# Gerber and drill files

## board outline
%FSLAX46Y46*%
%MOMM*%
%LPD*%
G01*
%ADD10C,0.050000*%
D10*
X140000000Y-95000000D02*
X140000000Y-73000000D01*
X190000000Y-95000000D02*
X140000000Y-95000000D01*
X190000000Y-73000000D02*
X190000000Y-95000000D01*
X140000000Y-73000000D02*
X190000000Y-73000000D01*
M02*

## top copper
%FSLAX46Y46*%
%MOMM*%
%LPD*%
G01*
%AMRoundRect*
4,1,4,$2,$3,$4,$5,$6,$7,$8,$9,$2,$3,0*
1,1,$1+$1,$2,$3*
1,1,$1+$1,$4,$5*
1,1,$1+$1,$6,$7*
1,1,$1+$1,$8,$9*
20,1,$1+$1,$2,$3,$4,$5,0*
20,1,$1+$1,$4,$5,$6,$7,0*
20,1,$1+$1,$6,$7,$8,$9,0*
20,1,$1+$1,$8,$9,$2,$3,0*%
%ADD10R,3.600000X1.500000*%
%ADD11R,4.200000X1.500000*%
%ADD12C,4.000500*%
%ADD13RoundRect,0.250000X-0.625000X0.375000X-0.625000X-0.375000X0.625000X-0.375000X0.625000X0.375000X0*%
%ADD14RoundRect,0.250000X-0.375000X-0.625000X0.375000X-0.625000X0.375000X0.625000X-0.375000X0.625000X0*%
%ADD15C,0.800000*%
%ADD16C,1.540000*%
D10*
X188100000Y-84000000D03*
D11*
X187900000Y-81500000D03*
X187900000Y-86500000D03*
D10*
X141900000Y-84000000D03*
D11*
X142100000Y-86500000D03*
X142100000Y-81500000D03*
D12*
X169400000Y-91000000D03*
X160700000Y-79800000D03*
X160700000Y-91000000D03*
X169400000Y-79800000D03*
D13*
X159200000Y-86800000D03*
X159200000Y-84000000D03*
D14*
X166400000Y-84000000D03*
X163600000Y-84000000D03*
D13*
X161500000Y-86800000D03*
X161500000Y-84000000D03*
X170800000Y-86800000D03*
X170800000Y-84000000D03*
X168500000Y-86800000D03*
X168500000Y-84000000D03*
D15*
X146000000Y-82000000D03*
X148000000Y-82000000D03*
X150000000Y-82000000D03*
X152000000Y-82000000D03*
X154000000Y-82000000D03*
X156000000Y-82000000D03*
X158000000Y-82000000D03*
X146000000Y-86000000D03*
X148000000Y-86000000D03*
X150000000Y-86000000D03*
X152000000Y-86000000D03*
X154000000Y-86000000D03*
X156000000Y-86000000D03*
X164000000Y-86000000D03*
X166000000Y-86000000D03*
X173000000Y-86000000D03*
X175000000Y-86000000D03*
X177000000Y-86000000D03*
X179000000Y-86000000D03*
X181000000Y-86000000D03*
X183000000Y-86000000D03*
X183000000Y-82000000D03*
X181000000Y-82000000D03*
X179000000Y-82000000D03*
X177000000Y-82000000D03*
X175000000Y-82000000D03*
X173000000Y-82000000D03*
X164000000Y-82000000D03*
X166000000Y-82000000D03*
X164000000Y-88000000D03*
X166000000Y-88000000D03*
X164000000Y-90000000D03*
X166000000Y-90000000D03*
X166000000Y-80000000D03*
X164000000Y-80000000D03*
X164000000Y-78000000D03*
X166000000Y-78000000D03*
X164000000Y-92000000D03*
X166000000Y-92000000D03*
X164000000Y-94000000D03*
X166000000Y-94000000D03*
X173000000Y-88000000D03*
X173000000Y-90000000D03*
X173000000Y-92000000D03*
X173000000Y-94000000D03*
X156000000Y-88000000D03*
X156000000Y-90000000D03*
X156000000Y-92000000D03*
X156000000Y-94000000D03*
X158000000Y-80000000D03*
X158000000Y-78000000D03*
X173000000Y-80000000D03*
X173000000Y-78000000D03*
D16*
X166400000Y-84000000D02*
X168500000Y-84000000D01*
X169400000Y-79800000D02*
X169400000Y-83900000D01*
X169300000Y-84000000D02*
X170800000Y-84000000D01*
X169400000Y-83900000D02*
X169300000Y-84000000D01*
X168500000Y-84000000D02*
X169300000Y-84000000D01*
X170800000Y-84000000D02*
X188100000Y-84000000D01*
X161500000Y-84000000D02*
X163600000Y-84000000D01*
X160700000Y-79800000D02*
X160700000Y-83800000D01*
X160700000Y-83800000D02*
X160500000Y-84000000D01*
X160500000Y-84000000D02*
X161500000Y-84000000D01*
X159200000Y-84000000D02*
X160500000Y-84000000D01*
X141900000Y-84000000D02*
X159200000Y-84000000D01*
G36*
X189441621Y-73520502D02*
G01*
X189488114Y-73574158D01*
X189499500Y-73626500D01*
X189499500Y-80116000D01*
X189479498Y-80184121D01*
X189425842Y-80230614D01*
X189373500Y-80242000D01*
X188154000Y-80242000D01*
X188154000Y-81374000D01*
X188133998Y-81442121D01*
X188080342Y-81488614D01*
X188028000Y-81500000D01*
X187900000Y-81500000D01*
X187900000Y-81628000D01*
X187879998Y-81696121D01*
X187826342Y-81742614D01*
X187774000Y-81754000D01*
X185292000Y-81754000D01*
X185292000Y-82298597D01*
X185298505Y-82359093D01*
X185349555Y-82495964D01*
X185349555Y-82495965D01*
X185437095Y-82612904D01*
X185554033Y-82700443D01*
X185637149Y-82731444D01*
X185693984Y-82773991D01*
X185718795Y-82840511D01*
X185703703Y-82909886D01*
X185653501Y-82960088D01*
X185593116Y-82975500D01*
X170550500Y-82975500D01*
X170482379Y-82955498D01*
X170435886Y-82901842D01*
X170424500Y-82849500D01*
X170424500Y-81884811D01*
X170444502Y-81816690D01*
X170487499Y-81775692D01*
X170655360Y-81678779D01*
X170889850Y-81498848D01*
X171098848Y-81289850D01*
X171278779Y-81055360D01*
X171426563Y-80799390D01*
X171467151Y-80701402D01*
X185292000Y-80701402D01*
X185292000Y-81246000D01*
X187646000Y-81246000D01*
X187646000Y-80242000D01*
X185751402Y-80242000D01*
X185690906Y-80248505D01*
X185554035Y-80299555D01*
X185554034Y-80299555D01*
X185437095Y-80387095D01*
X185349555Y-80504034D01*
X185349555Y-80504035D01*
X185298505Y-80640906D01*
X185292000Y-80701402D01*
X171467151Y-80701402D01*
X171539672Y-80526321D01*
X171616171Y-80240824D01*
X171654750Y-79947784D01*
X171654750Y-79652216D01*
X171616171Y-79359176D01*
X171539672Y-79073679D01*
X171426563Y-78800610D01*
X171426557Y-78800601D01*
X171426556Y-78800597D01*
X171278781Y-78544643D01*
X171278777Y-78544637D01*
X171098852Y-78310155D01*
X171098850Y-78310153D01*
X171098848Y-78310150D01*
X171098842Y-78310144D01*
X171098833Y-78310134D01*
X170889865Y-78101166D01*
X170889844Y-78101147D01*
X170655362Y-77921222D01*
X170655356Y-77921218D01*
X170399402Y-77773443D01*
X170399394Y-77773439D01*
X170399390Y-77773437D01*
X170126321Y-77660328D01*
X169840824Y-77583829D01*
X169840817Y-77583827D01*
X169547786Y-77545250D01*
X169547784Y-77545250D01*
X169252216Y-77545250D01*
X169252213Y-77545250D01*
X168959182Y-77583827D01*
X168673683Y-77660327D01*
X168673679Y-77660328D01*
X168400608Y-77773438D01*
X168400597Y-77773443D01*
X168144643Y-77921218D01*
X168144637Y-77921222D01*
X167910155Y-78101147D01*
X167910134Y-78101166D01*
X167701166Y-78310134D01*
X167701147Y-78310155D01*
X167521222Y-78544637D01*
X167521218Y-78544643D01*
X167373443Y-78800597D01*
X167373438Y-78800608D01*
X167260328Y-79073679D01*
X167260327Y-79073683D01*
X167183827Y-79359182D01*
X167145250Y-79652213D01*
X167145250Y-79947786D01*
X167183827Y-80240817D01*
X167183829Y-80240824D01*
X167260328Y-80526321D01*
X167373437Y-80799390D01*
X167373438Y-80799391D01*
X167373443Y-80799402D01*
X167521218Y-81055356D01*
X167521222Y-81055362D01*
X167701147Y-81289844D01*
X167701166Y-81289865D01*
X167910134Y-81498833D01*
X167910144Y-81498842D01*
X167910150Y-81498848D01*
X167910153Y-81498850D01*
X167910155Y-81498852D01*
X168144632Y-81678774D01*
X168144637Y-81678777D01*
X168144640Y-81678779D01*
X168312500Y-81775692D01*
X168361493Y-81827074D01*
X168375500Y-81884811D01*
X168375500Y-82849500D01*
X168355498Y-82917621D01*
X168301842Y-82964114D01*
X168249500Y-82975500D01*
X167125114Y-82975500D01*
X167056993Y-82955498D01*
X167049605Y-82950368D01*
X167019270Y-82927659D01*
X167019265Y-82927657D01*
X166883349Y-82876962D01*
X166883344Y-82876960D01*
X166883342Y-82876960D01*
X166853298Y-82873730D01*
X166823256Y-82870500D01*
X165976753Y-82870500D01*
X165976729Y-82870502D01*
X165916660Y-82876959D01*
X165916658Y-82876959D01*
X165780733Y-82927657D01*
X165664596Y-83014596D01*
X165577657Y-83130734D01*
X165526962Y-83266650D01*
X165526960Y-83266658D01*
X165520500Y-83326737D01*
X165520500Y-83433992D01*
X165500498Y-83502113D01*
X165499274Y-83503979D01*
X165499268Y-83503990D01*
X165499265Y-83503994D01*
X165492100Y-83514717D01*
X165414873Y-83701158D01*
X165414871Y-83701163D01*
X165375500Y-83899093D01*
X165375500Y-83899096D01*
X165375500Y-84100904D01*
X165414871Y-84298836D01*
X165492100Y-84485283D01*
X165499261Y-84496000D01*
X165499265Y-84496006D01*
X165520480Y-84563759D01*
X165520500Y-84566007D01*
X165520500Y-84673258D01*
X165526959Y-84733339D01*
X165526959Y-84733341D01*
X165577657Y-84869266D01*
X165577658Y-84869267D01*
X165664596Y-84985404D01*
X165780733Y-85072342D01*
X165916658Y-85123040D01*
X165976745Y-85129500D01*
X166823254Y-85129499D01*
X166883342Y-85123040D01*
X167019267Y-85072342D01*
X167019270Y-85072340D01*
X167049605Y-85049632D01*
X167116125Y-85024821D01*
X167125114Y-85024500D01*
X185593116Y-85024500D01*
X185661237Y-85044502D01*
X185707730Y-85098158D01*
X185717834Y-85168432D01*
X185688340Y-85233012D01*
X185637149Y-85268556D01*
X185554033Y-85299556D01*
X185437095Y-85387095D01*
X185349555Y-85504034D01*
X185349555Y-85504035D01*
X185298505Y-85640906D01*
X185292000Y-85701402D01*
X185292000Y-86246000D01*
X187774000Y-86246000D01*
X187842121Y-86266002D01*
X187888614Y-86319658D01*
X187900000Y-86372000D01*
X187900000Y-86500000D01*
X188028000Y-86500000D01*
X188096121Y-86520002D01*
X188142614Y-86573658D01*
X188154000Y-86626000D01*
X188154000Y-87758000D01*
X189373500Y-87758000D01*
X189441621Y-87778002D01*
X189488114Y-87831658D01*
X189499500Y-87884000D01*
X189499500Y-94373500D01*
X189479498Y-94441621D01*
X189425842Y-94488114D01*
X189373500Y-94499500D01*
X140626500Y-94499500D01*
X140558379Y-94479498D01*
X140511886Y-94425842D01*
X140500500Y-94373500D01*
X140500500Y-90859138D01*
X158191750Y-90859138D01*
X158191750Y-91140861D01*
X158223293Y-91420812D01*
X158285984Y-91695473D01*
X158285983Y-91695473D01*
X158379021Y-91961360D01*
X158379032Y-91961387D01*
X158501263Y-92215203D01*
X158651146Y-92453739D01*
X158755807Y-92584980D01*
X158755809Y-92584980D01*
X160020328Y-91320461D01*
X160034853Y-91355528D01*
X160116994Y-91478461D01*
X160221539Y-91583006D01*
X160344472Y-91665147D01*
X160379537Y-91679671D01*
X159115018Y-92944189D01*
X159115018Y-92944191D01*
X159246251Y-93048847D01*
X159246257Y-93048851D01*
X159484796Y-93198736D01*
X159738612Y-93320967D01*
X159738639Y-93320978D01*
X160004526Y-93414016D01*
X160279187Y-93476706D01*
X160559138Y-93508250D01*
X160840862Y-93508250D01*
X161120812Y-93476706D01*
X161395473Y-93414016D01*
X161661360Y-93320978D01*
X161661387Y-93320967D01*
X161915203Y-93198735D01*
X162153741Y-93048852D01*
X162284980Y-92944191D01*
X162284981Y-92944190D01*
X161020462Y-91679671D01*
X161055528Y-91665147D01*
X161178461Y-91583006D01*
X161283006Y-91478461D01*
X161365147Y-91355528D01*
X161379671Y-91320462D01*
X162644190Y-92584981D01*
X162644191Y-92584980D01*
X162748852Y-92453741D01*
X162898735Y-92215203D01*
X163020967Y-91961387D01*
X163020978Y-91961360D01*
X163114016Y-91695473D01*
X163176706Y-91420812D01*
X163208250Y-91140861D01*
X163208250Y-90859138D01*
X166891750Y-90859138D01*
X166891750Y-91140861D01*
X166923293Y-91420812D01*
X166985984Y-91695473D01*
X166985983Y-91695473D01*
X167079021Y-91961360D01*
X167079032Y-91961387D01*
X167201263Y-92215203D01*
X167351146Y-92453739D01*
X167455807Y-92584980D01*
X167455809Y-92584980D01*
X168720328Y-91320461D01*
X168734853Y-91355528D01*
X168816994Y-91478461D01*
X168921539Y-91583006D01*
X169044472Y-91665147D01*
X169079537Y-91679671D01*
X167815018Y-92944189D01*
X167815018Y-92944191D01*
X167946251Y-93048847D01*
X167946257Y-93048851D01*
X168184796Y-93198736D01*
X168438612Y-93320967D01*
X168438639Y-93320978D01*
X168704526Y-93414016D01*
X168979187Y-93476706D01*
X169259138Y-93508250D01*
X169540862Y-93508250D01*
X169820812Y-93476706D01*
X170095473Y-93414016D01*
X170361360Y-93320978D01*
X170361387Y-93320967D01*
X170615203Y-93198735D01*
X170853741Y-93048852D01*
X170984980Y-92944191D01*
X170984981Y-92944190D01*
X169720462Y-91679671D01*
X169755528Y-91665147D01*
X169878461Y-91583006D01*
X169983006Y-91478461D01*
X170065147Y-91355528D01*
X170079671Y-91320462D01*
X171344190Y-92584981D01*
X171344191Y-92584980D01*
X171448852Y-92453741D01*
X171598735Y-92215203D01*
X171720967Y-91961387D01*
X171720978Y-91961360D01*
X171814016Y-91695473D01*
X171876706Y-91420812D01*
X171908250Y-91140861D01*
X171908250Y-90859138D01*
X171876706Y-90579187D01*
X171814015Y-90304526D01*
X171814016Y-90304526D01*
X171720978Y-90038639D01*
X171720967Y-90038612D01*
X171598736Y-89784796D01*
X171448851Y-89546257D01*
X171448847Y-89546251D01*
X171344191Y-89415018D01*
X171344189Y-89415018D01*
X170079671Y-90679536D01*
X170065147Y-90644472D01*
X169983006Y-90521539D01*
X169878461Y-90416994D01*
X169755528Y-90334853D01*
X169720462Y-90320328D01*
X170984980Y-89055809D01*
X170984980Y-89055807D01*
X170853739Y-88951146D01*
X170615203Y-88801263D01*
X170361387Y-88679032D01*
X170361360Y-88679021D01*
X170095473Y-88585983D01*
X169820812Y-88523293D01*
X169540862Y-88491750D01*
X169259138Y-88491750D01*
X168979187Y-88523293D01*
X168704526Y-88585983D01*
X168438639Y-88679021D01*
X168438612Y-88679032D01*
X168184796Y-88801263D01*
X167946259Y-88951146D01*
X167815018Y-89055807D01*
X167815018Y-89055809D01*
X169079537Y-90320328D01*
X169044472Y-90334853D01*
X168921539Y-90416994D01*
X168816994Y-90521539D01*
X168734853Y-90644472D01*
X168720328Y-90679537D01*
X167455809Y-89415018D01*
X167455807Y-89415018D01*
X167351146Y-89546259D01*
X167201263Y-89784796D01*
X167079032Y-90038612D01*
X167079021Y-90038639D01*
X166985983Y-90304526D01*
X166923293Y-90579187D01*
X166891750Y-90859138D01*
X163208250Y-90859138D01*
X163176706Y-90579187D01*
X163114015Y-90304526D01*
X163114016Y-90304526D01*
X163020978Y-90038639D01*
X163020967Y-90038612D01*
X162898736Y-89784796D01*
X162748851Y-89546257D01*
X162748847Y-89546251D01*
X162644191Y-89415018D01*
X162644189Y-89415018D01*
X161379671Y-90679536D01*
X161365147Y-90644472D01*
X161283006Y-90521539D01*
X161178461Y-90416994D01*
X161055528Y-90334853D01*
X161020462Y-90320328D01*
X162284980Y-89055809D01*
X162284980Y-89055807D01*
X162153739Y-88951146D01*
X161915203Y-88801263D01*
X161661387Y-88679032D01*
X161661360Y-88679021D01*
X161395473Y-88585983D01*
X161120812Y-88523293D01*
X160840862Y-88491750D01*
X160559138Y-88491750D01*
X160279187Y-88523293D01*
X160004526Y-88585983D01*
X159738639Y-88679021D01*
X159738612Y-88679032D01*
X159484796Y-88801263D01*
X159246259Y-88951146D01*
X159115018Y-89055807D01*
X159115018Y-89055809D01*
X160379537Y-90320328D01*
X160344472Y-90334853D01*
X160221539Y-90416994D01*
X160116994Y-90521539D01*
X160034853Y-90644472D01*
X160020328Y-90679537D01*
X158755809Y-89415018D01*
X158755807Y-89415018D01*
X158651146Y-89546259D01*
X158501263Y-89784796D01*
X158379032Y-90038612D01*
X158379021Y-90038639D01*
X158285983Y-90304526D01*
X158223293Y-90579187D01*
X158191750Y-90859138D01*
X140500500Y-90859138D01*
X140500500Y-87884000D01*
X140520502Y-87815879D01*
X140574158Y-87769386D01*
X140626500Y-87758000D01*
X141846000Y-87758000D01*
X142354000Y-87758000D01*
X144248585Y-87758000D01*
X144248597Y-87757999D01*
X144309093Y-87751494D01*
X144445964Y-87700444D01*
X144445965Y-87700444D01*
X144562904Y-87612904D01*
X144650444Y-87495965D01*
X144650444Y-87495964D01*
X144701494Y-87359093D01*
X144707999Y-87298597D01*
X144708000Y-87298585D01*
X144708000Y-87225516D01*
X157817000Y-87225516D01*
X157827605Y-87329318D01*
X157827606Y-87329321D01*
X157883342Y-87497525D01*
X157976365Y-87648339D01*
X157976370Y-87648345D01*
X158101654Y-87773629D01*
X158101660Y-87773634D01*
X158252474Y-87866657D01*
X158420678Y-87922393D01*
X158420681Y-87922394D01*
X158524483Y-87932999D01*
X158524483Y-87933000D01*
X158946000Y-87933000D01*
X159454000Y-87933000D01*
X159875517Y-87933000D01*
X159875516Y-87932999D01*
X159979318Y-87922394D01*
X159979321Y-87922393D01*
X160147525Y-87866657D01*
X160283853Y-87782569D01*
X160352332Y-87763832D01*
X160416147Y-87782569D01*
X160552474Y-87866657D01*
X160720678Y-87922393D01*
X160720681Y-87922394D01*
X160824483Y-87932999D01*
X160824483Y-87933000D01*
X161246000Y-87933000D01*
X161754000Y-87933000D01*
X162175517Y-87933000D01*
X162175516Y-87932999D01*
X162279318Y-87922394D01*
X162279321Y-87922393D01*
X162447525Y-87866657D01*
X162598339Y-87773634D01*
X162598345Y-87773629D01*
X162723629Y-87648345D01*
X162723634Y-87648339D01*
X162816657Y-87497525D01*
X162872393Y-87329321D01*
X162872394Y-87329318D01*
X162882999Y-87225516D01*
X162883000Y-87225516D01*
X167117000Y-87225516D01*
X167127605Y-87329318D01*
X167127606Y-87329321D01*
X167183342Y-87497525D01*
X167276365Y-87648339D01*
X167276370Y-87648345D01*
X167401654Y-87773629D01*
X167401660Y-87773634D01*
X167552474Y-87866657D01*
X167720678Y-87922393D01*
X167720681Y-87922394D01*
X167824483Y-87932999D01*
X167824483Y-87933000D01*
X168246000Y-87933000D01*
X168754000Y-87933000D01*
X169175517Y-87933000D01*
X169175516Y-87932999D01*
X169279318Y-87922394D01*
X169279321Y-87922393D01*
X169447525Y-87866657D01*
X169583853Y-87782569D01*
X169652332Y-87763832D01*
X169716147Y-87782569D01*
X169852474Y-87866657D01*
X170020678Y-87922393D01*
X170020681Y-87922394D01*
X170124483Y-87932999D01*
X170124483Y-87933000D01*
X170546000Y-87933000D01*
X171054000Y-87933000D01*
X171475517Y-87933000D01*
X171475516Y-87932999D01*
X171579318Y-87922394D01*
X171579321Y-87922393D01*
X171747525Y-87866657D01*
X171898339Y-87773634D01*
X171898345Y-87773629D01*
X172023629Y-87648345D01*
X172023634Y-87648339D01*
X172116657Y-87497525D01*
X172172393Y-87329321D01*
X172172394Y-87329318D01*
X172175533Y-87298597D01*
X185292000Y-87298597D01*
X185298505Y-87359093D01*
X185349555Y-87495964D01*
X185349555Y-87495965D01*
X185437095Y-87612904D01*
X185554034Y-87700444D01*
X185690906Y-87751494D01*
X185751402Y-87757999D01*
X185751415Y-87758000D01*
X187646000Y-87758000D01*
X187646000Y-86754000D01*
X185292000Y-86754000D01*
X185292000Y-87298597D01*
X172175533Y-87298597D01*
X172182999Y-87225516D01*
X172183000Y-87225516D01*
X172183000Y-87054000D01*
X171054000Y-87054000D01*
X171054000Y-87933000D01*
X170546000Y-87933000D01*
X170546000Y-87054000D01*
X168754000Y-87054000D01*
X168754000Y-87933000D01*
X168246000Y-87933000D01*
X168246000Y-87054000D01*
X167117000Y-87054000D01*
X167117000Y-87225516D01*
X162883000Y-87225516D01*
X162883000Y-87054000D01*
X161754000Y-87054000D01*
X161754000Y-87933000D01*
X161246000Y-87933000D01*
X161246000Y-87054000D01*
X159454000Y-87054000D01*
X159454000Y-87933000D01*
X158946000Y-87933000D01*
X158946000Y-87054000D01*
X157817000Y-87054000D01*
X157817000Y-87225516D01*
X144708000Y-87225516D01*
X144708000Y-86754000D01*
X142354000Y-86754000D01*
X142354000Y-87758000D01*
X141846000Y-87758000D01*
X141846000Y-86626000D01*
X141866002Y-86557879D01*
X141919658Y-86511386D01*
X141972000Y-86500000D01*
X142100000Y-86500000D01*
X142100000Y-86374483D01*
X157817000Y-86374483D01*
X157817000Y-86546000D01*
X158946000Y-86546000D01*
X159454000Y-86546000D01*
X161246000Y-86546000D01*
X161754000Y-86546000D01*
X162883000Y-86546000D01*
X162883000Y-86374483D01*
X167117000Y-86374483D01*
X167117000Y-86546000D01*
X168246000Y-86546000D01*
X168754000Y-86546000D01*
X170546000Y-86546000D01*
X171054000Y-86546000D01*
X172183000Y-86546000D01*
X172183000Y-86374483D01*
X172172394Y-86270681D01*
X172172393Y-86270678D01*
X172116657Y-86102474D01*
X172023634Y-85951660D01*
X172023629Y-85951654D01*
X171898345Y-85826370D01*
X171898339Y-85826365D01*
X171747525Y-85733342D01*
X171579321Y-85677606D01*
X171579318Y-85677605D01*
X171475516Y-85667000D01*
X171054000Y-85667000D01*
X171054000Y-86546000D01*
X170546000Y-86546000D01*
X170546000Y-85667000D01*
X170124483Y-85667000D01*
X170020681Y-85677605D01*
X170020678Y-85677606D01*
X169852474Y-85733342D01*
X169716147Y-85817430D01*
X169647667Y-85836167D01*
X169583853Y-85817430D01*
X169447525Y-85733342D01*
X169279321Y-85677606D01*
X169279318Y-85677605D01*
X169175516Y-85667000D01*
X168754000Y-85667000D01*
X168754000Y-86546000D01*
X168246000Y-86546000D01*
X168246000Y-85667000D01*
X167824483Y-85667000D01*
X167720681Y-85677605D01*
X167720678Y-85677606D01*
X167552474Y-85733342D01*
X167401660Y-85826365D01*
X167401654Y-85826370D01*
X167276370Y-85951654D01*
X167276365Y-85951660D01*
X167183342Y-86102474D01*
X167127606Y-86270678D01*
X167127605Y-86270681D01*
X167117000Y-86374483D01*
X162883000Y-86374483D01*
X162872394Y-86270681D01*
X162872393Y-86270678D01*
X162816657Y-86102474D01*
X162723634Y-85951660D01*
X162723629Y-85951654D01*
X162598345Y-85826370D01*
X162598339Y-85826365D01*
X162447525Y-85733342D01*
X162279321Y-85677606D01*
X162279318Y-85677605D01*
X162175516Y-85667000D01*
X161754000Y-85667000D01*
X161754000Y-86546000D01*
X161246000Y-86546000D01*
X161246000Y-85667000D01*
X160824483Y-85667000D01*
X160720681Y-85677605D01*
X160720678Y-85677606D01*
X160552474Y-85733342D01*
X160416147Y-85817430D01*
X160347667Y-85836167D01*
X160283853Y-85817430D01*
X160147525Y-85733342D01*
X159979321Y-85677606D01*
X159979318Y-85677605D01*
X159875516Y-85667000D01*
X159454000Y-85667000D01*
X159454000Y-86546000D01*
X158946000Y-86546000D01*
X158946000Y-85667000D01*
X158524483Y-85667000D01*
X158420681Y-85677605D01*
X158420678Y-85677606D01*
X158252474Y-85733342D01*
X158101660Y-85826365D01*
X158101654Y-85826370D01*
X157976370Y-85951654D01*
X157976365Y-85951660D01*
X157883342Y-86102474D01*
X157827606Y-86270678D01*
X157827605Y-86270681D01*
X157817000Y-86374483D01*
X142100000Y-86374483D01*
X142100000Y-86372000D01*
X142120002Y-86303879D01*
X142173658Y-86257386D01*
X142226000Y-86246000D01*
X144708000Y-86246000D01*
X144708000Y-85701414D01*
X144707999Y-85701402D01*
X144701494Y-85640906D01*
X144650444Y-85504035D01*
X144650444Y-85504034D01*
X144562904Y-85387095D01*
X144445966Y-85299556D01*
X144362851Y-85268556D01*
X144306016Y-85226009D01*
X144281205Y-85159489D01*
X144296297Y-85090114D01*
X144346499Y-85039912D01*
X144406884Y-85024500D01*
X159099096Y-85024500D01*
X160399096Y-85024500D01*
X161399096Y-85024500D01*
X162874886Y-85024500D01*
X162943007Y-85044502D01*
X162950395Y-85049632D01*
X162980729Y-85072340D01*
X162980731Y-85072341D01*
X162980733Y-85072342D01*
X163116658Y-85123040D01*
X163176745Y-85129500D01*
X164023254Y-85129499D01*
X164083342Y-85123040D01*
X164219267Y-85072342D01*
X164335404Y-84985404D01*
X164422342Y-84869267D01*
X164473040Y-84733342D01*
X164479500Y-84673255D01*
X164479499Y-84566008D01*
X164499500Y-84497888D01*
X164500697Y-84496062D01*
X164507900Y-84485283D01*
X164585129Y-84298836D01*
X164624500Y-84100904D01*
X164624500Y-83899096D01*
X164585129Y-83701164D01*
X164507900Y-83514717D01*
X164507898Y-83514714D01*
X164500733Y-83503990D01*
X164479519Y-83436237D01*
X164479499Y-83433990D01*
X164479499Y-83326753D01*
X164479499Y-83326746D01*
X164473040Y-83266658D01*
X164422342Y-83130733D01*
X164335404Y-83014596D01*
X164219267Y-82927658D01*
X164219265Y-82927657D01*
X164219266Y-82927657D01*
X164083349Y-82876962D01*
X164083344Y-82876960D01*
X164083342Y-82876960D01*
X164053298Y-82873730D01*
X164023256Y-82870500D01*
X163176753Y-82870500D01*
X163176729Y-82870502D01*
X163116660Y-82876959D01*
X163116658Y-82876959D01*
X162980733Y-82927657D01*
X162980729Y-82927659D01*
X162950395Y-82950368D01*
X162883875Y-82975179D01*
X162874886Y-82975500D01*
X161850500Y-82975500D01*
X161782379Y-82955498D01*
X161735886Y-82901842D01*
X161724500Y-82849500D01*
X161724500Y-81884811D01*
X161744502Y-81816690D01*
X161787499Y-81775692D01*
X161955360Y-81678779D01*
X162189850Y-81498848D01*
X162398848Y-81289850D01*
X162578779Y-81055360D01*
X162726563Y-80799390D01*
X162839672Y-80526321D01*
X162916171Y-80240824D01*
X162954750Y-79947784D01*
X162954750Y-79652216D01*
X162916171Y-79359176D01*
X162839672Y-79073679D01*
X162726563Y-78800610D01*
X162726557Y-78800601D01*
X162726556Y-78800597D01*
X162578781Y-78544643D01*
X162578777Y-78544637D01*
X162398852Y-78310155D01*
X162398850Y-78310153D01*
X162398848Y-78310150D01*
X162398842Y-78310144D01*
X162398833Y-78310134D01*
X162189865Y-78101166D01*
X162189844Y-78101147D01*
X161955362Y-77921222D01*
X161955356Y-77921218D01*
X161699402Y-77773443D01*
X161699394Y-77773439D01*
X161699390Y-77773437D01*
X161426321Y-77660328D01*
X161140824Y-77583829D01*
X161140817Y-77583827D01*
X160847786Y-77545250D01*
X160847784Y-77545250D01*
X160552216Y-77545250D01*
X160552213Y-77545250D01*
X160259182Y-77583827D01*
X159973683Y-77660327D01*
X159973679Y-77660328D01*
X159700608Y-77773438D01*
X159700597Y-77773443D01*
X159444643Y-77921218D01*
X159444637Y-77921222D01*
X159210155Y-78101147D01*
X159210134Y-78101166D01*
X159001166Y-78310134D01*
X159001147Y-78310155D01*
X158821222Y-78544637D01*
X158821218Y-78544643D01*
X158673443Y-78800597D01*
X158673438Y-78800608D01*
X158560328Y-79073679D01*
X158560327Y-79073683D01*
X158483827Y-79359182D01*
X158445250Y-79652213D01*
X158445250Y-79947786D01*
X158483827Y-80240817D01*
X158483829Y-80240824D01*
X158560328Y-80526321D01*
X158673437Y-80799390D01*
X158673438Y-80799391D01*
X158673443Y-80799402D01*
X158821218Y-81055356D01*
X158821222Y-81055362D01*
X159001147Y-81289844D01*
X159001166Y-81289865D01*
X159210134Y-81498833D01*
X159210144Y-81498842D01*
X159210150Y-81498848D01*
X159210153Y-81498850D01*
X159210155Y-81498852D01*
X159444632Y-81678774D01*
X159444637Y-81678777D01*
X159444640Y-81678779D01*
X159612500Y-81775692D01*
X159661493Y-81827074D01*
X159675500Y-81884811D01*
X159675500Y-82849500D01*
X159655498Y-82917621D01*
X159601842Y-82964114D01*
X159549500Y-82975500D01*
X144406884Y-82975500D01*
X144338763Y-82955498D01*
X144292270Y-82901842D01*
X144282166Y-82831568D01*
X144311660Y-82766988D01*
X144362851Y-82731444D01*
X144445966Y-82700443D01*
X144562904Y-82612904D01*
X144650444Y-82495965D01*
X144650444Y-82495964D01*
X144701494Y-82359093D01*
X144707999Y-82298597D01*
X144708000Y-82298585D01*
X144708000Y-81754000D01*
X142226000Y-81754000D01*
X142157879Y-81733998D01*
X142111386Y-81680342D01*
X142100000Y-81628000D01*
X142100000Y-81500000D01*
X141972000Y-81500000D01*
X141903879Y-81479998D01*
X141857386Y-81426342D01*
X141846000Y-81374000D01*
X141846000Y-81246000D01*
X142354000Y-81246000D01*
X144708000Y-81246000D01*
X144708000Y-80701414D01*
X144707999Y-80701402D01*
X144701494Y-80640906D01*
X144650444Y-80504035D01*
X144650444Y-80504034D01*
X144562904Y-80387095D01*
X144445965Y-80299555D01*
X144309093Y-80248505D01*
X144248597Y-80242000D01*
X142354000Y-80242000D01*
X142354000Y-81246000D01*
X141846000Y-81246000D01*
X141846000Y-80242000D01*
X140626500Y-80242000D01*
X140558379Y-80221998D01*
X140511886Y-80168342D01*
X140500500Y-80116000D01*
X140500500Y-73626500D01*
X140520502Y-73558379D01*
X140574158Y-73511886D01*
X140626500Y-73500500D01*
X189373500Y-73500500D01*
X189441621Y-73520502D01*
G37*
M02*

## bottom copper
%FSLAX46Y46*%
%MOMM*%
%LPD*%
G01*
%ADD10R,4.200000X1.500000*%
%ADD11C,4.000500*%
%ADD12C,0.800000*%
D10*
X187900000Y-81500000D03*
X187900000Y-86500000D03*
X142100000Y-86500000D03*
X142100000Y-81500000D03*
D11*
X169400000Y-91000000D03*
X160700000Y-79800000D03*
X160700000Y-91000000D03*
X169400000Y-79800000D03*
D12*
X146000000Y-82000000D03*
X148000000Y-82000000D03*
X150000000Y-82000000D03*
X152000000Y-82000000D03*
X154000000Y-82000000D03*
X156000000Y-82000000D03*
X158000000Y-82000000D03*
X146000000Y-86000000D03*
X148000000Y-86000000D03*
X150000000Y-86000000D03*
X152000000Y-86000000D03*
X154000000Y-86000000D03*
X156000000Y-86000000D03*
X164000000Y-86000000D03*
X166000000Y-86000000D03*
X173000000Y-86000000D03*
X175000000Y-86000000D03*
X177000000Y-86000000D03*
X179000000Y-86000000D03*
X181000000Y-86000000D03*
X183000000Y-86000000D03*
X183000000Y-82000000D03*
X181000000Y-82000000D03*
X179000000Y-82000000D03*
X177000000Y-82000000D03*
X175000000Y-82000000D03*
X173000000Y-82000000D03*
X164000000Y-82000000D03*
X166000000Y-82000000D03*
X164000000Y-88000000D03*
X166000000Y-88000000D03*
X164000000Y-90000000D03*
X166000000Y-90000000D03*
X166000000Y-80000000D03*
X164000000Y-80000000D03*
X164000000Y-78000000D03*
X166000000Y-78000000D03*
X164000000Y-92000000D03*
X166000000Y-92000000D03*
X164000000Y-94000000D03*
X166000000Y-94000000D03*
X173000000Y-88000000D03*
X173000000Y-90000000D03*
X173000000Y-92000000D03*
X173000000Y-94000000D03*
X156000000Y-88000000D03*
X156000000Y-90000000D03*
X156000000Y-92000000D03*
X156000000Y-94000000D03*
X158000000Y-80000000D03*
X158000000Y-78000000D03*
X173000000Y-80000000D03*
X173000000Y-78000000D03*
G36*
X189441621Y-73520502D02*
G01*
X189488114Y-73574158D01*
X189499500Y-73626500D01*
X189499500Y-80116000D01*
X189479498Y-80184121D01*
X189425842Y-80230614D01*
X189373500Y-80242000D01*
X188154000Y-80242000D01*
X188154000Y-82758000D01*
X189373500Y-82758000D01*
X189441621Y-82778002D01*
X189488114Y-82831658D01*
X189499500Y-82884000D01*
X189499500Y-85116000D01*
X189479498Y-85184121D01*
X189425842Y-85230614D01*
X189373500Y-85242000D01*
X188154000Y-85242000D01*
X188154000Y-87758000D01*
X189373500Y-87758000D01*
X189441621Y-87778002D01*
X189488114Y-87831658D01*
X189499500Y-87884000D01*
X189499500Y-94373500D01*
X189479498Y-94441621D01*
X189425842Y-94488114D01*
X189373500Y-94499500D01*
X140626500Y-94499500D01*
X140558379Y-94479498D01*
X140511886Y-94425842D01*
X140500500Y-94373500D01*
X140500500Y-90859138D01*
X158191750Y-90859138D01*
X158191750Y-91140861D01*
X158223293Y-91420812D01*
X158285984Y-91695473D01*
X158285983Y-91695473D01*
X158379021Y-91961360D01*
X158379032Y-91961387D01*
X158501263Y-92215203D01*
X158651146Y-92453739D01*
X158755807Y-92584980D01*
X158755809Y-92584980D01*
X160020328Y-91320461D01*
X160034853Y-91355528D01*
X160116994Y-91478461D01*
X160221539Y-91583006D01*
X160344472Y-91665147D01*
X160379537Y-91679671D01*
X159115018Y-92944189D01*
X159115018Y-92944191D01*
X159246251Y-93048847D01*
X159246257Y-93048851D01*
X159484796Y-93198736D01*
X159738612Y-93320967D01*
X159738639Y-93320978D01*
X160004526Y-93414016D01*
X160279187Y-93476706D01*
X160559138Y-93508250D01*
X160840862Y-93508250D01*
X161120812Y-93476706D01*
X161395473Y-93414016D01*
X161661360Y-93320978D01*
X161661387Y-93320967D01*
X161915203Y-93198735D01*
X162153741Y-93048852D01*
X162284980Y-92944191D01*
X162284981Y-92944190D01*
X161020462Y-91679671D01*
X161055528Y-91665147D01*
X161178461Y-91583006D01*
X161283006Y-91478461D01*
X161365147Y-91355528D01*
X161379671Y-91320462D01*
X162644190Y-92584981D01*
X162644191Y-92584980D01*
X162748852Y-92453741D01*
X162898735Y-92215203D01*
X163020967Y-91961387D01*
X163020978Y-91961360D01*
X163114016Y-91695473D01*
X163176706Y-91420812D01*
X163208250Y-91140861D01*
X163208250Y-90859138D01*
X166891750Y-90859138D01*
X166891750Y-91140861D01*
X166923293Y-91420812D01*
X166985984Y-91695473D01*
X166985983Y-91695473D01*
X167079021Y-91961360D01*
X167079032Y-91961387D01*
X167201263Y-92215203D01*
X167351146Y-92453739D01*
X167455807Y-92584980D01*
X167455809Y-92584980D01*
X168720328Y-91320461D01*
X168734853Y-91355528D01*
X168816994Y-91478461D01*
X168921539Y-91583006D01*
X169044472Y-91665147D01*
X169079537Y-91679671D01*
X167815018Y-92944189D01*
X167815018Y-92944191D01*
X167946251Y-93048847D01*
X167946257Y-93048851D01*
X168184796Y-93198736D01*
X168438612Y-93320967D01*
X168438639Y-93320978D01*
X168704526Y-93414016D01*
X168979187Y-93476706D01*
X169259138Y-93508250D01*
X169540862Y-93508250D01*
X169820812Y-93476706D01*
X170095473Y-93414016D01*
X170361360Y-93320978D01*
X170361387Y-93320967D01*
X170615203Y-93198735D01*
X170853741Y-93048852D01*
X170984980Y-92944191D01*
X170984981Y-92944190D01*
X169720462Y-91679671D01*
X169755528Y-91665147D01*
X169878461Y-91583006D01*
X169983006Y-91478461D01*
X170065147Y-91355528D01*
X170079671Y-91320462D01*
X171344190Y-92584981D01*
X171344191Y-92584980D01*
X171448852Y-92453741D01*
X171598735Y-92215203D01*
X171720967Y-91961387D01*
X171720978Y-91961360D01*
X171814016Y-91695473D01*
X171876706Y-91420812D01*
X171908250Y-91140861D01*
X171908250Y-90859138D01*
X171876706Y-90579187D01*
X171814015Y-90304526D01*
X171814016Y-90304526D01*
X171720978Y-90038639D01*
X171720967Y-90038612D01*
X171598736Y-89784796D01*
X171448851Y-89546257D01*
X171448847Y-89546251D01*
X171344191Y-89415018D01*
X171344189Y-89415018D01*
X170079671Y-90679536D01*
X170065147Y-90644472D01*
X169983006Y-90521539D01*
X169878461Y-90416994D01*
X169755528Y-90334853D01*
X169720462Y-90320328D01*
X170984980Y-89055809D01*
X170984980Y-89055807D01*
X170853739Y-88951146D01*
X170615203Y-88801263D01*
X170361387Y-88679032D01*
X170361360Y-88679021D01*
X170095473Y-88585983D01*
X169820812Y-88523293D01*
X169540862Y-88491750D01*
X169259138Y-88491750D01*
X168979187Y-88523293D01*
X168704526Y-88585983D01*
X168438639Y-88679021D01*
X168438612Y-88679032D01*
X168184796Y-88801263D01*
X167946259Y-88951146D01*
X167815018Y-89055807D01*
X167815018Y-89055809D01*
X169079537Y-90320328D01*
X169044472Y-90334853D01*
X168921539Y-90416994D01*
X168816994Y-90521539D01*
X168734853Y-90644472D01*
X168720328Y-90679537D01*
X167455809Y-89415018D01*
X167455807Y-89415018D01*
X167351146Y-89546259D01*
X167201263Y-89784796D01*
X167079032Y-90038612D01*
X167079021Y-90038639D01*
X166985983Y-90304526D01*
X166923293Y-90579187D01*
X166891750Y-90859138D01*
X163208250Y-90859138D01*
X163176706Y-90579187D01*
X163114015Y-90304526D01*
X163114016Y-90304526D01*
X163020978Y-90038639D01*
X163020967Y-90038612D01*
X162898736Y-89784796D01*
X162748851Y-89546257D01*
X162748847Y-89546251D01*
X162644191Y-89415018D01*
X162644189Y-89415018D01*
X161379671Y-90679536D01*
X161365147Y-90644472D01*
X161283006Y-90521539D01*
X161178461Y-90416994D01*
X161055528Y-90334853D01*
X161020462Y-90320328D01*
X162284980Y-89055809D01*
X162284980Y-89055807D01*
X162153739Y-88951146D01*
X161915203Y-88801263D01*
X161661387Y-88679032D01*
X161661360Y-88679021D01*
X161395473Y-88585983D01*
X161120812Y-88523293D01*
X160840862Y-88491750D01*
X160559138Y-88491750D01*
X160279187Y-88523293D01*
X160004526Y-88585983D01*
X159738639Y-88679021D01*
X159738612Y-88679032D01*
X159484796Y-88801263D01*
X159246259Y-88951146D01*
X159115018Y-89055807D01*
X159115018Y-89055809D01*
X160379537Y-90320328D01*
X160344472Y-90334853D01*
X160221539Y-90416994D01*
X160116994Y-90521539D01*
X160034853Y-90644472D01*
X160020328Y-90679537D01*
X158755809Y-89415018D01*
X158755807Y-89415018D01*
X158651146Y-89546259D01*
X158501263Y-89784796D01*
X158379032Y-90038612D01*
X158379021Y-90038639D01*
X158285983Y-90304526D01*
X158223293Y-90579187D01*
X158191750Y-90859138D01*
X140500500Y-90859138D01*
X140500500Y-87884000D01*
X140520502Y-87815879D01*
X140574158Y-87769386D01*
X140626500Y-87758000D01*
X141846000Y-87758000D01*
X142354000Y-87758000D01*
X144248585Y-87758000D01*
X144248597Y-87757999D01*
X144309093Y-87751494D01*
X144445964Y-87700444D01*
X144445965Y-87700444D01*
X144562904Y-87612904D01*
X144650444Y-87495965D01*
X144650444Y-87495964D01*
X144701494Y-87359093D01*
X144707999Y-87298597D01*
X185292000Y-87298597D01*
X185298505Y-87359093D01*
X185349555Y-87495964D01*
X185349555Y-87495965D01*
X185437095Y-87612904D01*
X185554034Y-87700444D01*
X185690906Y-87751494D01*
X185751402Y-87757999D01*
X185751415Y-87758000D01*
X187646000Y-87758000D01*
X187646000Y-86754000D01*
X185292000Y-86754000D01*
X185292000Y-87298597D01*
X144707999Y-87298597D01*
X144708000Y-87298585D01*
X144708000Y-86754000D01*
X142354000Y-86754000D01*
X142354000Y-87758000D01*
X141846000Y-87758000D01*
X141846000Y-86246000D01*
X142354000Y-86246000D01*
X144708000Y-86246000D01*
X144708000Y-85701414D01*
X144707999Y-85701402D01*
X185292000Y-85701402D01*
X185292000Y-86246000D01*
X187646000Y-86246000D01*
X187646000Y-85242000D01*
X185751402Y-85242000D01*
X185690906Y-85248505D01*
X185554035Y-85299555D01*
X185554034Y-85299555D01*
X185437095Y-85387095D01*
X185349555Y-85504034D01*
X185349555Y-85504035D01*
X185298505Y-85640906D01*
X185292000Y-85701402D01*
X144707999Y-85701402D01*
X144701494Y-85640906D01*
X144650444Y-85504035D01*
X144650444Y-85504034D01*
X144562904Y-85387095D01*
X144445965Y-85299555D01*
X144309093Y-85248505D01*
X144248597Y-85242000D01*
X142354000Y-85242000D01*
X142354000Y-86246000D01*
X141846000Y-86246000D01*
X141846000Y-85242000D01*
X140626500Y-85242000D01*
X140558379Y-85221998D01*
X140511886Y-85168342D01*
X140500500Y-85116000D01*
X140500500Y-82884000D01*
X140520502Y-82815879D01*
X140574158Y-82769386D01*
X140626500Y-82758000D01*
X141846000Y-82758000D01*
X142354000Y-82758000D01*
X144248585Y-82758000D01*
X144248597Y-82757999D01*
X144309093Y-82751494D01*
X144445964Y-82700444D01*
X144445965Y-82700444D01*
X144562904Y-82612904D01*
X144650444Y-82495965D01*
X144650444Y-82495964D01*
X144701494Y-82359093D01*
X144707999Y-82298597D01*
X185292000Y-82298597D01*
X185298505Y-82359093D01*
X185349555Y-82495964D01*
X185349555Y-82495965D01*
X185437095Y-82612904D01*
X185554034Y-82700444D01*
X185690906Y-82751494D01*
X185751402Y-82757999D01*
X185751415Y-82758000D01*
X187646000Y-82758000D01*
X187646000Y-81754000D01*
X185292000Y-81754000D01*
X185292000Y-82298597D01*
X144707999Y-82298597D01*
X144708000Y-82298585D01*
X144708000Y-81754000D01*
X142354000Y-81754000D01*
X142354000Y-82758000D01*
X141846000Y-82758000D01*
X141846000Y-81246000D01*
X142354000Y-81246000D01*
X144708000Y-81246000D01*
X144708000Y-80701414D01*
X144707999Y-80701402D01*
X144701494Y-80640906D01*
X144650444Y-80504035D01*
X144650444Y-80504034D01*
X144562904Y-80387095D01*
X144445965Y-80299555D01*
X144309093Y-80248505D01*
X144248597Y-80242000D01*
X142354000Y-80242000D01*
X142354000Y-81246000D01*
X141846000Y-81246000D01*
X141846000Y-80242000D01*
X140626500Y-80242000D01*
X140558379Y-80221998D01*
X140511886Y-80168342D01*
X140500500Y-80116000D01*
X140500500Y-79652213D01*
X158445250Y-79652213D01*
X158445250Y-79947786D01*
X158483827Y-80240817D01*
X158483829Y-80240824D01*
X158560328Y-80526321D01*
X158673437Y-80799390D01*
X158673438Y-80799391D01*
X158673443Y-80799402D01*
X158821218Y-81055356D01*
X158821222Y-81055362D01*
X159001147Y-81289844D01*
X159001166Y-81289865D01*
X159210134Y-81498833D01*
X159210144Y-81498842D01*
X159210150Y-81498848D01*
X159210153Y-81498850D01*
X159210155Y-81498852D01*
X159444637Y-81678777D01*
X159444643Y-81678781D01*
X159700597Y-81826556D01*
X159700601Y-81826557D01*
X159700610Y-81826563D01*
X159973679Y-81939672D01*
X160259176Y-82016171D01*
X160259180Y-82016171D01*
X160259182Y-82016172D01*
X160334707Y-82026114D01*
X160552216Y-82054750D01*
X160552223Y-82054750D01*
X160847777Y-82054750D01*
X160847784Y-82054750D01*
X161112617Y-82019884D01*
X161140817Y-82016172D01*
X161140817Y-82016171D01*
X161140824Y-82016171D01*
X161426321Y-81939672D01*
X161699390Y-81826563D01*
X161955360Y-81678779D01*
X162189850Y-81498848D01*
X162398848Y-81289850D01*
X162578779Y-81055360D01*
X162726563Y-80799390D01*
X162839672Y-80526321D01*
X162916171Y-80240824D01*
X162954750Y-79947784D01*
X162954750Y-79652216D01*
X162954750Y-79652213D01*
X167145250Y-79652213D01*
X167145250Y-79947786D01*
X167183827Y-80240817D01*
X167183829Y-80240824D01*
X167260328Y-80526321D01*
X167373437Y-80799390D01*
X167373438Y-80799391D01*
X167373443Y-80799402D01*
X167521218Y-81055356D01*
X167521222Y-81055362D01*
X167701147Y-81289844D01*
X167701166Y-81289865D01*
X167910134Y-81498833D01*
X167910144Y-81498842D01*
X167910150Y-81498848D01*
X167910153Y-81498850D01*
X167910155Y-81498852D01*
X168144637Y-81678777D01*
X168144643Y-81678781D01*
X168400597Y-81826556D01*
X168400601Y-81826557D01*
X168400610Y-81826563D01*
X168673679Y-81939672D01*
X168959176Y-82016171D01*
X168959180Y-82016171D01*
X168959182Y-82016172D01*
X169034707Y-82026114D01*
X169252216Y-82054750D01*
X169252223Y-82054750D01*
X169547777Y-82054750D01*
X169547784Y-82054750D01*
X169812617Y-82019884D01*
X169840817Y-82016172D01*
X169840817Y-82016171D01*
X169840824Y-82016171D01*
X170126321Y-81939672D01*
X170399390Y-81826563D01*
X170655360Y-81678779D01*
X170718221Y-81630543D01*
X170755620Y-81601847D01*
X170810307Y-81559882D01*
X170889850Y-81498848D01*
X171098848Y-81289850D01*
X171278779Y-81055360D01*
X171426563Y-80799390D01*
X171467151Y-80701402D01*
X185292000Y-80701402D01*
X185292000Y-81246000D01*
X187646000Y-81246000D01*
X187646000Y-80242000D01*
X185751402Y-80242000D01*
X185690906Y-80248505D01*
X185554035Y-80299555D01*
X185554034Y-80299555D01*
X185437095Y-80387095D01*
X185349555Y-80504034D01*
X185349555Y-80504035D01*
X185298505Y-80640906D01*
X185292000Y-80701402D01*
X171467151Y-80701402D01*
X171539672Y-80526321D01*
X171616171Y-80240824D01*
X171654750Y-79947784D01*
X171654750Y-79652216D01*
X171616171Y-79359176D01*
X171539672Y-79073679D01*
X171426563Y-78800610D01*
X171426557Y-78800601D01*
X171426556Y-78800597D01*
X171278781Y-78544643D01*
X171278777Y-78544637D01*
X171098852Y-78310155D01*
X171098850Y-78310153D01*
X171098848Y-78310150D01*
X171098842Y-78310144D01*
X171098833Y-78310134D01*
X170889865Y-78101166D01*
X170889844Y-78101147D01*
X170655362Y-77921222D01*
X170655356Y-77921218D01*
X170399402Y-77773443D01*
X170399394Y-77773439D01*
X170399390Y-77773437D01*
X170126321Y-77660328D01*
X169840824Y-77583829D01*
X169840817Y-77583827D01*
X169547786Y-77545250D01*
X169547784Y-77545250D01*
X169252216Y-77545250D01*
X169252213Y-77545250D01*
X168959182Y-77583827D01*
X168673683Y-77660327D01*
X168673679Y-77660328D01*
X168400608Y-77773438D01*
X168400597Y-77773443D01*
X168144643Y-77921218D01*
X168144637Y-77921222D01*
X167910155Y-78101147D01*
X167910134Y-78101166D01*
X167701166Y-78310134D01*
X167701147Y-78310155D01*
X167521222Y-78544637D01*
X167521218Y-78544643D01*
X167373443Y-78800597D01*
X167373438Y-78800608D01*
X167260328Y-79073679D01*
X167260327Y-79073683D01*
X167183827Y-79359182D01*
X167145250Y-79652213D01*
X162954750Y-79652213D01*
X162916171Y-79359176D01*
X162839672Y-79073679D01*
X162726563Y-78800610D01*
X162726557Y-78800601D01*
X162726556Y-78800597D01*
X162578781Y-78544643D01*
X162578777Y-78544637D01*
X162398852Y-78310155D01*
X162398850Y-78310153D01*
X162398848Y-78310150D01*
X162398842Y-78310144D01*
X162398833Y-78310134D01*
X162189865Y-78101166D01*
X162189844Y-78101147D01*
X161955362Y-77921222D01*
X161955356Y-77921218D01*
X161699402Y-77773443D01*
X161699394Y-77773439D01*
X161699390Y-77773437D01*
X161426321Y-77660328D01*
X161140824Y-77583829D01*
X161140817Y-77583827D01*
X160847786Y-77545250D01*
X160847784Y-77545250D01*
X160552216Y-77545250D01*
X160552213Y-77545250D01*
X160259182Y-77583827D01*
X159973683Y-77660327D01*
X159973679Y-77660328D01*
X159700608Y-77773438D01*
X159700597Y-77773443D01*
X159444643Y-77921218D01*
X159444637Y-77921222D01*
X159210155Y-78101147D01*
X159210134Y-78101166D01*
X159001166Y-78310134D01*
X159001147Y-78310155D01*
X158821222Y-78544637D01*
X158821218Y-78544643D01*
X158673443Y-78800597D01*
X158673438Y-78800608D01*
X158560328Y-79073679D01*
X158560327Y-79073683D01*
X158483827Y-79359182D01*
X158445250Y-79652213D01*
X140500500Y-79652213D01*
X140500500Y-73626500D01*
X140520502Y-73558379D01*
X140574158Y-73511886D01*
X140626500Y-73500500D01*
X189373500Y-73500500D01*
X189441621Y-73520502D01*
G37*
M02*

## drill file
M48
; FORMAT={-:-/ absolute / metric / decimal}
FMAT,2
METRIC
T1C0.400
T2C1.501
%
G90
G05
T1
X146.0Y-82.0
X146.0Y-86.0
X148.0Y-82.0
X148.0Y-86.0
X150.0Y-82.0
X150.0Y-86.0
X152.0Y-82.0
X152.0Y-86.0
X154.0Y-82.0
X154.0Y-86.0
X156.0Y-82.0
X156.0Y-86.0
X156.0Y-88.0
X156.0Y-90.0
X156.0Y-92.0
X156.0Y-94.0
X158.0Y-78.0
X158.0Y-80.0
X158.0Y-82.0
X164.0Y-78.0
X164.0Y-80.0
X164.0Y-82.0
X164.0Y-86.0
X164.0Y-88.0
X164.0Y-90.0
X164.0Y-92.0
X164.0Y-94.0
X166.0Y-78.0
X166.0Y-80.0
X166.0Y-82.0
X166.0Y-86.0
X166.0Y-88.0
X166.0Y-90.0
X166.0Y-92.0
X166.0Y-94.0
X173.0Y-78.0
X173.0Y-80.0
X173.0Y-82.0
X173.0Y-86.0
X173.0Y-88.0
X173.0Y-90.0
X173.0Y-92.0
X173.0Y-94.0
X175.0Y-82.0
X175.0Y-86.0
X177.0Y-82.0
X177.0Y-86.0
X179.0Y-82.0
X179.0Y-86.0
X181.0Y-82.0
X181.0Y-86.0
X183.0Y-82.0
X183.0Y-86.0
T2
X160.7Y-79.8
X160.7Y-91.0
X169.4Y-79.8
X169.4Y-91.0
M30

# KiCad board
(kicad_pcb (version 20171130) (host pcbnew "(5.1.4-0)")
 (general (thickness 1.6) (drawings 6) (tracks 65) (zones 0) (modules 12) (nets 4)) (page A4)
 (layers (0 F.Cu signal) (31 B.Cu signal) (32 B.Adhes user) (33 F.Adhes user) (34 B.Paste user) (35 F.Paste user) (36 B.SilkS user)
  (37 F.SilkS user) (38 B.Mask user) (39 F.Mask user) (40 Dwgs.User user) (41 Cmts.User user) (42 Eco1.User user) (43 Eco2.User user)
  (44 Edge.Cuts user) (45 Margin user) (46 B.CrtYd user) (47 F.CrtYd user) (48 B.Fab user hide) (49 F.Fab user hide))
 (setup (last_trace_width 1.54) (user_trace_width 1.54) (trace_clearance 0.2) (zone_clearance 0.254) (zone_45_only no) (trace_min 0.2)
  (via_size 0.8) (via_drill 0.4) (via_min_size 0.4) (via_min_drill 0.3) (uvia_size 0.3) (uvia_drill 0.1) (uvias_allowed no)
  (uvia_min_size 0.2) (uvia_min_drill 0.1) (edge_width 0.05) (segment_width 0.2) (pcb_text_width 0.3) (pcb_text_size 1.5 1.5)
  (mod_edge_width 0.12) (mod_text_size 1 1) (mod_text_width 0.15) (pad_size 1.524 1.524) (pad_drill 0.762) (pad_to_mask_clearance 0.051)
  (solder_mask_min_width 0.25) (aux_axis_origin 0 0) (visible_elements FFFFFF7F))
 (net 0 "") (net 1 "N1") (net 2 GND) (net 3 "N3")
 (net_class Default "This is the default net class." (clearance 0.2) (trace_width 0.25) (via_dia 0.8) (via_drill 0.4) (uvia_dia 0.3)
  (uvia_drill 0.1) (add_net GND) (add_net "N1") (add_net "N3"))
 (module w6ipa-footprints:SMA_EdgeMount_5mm (layer F.Cu) (at 187.9 84)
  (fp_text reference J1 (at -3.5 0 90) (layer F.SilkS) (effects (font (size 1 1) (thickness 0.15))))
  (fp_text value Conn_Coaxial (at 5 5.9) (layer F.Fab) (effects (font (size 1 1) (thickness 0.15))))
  (pad 1 smd rect (at 0.2 0 90) (size 1.5 3.6) (layers F.Cu F.Paste F.Mask) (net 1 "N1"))
  (pad 2 smd rect (at 0 -2.5 90) (size 1.5 4.2) (layers F.Cu F.Paste F.Mask) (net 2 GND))
  (pad 2 smd rect (at 0 2.5 90) (size 1.5 4.2) (layers F.Cu F.Paste F.Mask) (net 2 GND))
  (pad 2 smd rect (at 0 -2.5 90) (size 1.5 4.2) (layers B.Cu B.Paste B.Mask) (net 2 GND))
  (pad 2 smd rect (at 0 2.5 90) (size 1.5 4.2) (layers B.Cu B.Paste B.Mask) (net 2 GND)))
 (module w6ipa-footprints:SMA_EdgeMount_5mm (layer F.Cu) (at 142.1 84 180)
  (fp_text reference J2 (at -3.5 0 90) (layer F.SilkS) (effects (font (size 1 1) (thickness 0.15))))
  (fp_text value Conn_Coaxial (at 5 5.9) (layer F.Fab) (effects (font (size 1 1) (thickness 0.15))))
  (pad 1 smd rect (at 0.2 0 270) (size 1.5 3.6) (layers F.Cu F.Paste F.Mask) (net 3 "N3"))
  (pad 2 smd rect (at 0 -2.5 270) (size 1.5 4.2) (layers F.Cu F.Paste F.Mask) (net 2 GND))
  (pad 2 smd rect (at 0 2.5 270) (size 1.5 4.2) (layers F.Cu F.Paste F.Mask) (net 2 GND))
  (pad 2 smd rect (at 0 -2.5 270) (size 1.5 4.2) (layers B.Cu B.Paste B.Mask) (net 2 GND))
  (pad 2 smd rect (at 0 2.5 270) (size 1.5 4.2) (layers B.Cu B.Paste B.Mask) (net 2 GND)))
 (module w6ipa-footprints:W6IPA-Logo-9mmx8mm (layer B.Cu) (at 165.5 85.25)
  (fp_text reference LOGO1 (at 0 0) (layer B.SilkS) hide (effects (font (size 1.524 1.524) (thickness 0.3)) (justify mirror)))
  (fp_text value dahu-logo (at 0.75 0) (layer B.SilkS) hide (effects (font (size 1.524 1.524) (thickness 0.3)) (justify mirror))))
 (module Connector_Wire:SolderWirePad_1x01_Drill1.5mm (layer F.Cu) (at 169.4 91)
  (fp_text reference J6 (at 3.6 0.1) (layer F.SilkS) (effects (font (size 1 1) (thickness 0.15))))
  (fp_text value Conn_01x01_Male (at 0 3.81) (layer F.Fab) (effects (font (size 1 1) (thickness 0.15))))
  (pad 1 thru_hole circle (at 0 0) (size 4.0005 4.0005) (drill 1.50114) (layers *.Cu *.Mask) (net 2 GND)))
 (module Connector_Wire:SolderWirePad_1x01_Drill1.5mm (layer F.Cu) (at 160.7 79.8)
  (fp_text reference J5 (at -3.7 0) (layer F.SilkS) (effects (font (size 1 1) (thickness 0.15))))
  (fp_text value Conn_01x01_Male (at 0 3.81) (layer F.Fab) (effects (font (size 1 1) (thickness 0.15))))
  (pad 1 thru_hole circle (at 0 0) (size 4.0005 4.0005) (drill 1.50114) (layers *.Cu *.Mask) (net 3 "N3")))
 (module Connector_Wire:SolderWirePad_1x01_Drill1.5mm (layer F.Cu) (at 160.7 91)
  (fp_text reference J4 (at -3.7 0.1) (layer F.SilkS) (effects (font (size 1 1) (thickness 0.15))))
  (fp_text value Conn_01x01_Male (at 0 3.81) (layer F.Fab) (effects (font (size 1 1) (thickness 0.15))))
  (pad 1 thru_hole circle (at 0 0) (size 4.0005 4.0005) (drill 1.50114) (layers *.Cu *.Mask) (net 2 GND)))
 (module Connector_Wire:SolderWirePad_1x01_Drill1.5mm (layer F.Cu) (at 169.4 79.8)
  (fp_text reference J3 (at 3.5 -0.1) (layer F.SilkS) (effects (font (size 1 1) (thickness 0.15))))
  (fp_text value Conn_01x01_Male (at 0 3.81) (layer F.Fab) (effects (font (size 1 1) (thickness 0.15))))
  (pad 1 thru_hole circle (at 0 0) (size 4.0005 4.0005) (drill 1.50114) (layers *.Cu *.Mask) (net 1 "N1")))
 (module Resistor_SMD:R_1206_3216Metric (layer F.Cu) (at 159.2 85.4 270)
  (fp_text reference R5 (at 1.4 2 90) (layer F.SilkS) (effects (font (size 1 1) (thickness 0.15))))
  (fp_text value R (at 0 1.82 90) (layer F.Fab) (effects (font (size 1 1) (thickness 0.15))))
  (pad 2 smd roundrect (at 1.4 0 270) (size 1.25 1.75) (layers F.Cu F.Paste F.Mask) (roundrect_rratio 0.2) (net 2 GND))
  (pad 1 smd roundrect (at -1.4 0 270) (size 1.25 1.75) (layers F.Cu F.Paste F.Mask) (roundrect_rratio 0.2) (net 3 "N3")))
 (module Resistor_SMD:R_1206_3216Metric (layer F.Cu) (at 165 84)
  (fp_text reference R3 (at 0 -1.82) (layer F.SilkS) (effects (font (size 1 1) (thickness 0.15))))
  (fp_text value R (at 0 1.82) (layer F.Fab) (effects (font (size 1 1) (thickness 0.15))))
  (pad 2 smd roundrect (at 1.4 0) (size 1.25 1.75) (layers F.Cu F.Paste F.Mask) (roundrect_rratio 0.2) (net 1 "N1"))
  (pad 1 smd roundrect (at -1.4 0) (size 1.25 1.75) (layers F.Cu F.Paste F.Mask) (roundrect_rratio 0.2) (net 3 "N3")))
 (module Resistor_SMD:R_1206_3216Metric (layer F.Cu) (at 161.5 85.4 270)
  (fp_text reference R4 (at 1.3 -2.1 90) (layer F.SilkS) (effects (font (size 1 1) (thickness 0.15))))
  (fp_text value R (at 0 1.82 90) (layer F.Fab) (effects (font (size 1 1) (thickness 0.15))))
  (pad 2 smd roundrect (at 1.4 0 270) (size 1.25 1.75) (layers F.Cu F.Paste F.Mask) (roundrect_rratio 0.2) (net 2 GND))
  (pad 1 smd roundrect (at -1.4 0 270) (size 1.25 1.75) (layers F.Cu F.Paste F.Mask) (roundrect_rratio 0.2) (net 3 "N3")))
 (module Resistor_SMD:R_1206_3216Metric (layer F.Cu) (at 170.8 85.4 270)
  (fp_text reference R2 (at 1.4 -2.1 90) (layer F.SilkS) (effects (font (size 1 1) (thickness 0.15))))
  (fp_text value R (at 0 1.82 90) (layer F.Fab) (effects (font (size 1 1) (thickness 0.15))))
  (pad 2 smd roundrect (at 1.4 0 270) (size 1.25 1.75) (layers F.Cu F.Paste F.Mask) (roundrect_rratio 0.2) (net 2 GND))
  (pad 1 smd roundrect (at -1.4 0 270) (size 1.25 1.75) (layers F.Cu F.Paste F.Mask) (roundrect_rratio 0.2) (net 1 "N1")))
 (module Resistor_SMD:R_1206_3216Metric (layer F.Cu) (at 168.5 85.4 270)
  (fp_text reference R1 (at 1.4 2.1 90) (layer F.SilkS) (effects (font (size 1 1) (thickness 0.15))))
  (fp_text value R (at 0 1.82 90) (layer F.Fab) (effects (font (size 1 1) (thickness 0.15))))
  (pad 2 smd roundrect (at 1.4 0 270) (size 1.25 1.75) (layers F.Cu F.Paste F.Mask) (roundrect_rratio 0.2) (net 2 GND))
  (pad 1 smd roundrect (at -1.4 0 270) (size 1.25 1.75) (layers F.Cu F.Paste F.Mask) (roundrect_rratio 0.2) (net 1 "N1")))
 (gr_line (start 140 95) (end 140 73) (layer Edge.Cuts) (width 0.05))
 (gr_line (start 190 95) (end 140 95) (layer Edge.Cuts) (width 0.05))
 (gr_line (start 190 73) (end 190 95) (layer Edge.Cuts) (width 0.05))
 (gr_line (start 140 73) (end 190 73) (layer Edge.Cuts) (width 0.05))
 (segment (start 166.4 84) (end 168.5 84) (width 1.54) (layer F.Cu) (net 1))
 (segment (start 169.4 79.8) (end 169.4 83.9) (width 1.54) (layer F.Cu) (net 1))
 (segment (start 169.3 84) (end 170.8 84) (width 1.54) (layer F.Cu) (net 1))
 (segment (start 169.4 83.9) (end 169.3 84) (width 1.54) (layer F.Cu) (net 1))
 (segment (start 168.5 84) (end 169.3 84) (width 1.54) (layer F.Cu) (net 1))
 (segment (start 170.8 84) (end 188.1 84) (width 1.54) (layer F.Cu) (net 1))
 (via (at 146 82) (size 0.8) (drill 0.4) (layers F.Cu B.Cu) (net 2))
 (via (at 148 82) (size 0.8) (drill 0.4) (layers F.Cu B.Cu) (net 2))
 (via (at 150 82) (size 0.8) (drill 0.4) (layers F.Cu B.Cu) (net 2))
 (via (at 152 82) (size 0.8) (drill 0.4) (layers F.Cu B.Cu) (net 2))
 (via (at 154 82) (size 0.8) (drill 0.4) (layers F.Cu B.Cu) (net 2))
 (via (at 156 82) (size 0.8) (drill 0.4) (layers F.Cu B.Cu) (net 2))
 (via (at 158 82) (size 0.8) (drill 0.4) (layers F.Cu B.Cu) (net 2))
 (via (at 146 86) (size 0.8) (drill 0.4) (layers F.Cu B.Cu) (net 2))
 (via (at 148 86) (size 0.8) (drill 0.4) (layers F.Cu B.Cu) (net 2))
 (via (at 150 86) (size 0.8) (drill 0.4) (layers F.Cu B.Cu) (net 2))
 (via (at 152 86) (size 0.8) (drill 0.4) (layers F.Cu B.Cu) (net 2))
 (via (at 154 86) (size 0.8) (drill 0.4) (layers F.Cu B.Cu) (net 2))
 (via (at 156 86) (size 0.8) (drill 0.4) (layers F.Cu B.Cu) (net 2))
 (via (at 164 86) (size 0.8) (drill 0.4) (layers F.Cu B.Cu) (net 2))
 (via (at 166 86) (size 0.8) (drill 0.4) (layers F.Cu B.Cu) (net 2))
 (via (at 173 86) (size 0.8) (drill 0.4) (layers F.Cu B.Cu) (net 2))
 (via (at 175 86) (size 0.8) (drill 0.4) (layers F.Cu B.Cu) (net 2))
 (via (at 177 86) (size 0.8) (drill 0.4) (layers F.Cu B.Cu) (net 2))
 (via (at 179 86) (size 0.8) (drill 0.4) (layers F.Cu B.Cu) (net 2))
 (via (at 181 86) (size 0.8) (drill 0.4) (layers F.Cu B.Cu) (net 2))
 (via (at 183 86) (size 0.8) (drill 0.4) (layers F.Cu B.Cu) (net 2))
 (via (at 183 82) (size 0.8) (drill 0.4) (layers F.Cu B.Cu) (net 2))
 (via (at 181 82) (size 0.8) (drill 0.4) (layers F.Cu B.Cu) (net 2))
 (via (at 179 82) (size 0.8) (drill 0.4) (layers F.Cu B.Cu) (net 2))
 (via (at 177 82) (size 0.8) (drill 0.4) (layers F.Cu B.Cu) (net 2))
 (via (at 175 82) (size 0.8) (drill 0.4) (layers F.Cu B.Cu) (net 2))
 (via (at 173 82) (size 0.8) (drill 0.4) (layers F.Cu B.Cu) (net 2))
 (via (at 164 82) (size 0.8) (drill 0.4) (layers F.Cu B.Cu) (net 2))
 (via (at 166 82) (size 0.8) (drill 0.4) (layers F.Cu B.Cu) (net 2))
 (via (at 164 88) (size 0.8) (drill 0.4) (layers F.Cu B.Cu) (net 2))
 (via (at 166 88) (size 0.8) (drill 0.4) (layers F.Cu B.Cu) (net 2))
 (via (at 164 90) (size 0.8) (drill 0.4) (layers F.Cu B.Cu) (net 2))
 (via (at 166 90) (size 0.8) (drill 0.4) (layers F.Cu B.Cu) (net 2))
 (via (at 166 80) (size 0.8) (drill 0.4) (layers F.Cu B.Cu) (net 2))
 (via (at 164 80) (size 0.8) (drill 0.4) (layers F.Cu B.Cu) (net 2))
 (via (at 164 78) (size 0.8) (drill 0.4) (layers F.Cu B.Cu) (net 2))
 (via (at 166 78) (size 0.8) (drill 0.4) (layers F.Cu B.Cu) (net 2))
 (via (at 164 92) (size 0.8) (drill 0.4) (layers F.Cu B.Cu) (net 2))
 (via (at 166 92) (size 0.8) (drill 0.4) (layers F.Cu B.Cu) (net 2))
 (via (at 164 94) (size 0.8) (drill 0.4) (layers F.Cu B.Cu) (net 2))
 (via (at 166 94) (size 0.8) (drill 0.4) (layers F.Cu B.Cu) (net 2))
 (via (at 173 88) (size 0.8) (drill 0.4) (layers F.Cu B.Cu) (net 2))
 (via (at 173 90) (size 0.8) (drill 0.4) (layers F.Cu B.Cu) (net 2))
 (via (at 173 92) (size 0.8) (drill 0.4) (layers F.Cu B.Cu) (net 2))
 (via (at 173 94) (size 0.8) (drill 0.4) (layers F.Cu B.Cu) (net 2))
 (via (at 156 88) (size 0.8) (drill 0.4) (layers F.Cu B.Cu) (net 2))
 (via (at 156 90) (size 0.8) (drill 0.4) (layers F.Cu B.Cu) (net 2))
 (via (at 156 92) (size 0.8) (drill 0.4) (layers F.Cu B.Cu) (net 2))
 (via (at 156 94) (size 0.8) (drill 0.4) (layers F.Cu B.Cu) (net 2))
 (via (at 158 80) (size 0.8) (drill 0.4) (layers F.Cu B.Cu) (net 2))
 (via (at 158 78) (size 0.8) (drill 0.4) (layers F.Cu B.Cu) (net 2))
 (via (at 173 80) (size 0.8) (drill 0.4) (layers F.Cu B.Cu) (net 2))
 (via (at 173 78) (size 0.8) (drill 0.4) (layers F.Cu B.Cu) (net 2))
 (segment (start 161.5 84) (end 163.6 84) (width 1.54) (layer F.Cu) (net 3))
 (segment (start 160.7 79.8) (end 160.7 83.8) (width 1.54) (layer F.Cu) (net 3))
 (segment (start 160.7 83.8) (end 160.5 84) (width 1.54) (layer F.Cu) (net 3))
 (segment (start 160.5 84) (end 161.5 84) (width 1.54) (layer F.Cu) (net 3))
 (segment (start 159.2 84) (end 160.5 84) (width 1.54) (layer F.Cu) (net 3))
 (segment (start 141.9 84) (end 159.2 84) (width 1.54) (layer F.Cu) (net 3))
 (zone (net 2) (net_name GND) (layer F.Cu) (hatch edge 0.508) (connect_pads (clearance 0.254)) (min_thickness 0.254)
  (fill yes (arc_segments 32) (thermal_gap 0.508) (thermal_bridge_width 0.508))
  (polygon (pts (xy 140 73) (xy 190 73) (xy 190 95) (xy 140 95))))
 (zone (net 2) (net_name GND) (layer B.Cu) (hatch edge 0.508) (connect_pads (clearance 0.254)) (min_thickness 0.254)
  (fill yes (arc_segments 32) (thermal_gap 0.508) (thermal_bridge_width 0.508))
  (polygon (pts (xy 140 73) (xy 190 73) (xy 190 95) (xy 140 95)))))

